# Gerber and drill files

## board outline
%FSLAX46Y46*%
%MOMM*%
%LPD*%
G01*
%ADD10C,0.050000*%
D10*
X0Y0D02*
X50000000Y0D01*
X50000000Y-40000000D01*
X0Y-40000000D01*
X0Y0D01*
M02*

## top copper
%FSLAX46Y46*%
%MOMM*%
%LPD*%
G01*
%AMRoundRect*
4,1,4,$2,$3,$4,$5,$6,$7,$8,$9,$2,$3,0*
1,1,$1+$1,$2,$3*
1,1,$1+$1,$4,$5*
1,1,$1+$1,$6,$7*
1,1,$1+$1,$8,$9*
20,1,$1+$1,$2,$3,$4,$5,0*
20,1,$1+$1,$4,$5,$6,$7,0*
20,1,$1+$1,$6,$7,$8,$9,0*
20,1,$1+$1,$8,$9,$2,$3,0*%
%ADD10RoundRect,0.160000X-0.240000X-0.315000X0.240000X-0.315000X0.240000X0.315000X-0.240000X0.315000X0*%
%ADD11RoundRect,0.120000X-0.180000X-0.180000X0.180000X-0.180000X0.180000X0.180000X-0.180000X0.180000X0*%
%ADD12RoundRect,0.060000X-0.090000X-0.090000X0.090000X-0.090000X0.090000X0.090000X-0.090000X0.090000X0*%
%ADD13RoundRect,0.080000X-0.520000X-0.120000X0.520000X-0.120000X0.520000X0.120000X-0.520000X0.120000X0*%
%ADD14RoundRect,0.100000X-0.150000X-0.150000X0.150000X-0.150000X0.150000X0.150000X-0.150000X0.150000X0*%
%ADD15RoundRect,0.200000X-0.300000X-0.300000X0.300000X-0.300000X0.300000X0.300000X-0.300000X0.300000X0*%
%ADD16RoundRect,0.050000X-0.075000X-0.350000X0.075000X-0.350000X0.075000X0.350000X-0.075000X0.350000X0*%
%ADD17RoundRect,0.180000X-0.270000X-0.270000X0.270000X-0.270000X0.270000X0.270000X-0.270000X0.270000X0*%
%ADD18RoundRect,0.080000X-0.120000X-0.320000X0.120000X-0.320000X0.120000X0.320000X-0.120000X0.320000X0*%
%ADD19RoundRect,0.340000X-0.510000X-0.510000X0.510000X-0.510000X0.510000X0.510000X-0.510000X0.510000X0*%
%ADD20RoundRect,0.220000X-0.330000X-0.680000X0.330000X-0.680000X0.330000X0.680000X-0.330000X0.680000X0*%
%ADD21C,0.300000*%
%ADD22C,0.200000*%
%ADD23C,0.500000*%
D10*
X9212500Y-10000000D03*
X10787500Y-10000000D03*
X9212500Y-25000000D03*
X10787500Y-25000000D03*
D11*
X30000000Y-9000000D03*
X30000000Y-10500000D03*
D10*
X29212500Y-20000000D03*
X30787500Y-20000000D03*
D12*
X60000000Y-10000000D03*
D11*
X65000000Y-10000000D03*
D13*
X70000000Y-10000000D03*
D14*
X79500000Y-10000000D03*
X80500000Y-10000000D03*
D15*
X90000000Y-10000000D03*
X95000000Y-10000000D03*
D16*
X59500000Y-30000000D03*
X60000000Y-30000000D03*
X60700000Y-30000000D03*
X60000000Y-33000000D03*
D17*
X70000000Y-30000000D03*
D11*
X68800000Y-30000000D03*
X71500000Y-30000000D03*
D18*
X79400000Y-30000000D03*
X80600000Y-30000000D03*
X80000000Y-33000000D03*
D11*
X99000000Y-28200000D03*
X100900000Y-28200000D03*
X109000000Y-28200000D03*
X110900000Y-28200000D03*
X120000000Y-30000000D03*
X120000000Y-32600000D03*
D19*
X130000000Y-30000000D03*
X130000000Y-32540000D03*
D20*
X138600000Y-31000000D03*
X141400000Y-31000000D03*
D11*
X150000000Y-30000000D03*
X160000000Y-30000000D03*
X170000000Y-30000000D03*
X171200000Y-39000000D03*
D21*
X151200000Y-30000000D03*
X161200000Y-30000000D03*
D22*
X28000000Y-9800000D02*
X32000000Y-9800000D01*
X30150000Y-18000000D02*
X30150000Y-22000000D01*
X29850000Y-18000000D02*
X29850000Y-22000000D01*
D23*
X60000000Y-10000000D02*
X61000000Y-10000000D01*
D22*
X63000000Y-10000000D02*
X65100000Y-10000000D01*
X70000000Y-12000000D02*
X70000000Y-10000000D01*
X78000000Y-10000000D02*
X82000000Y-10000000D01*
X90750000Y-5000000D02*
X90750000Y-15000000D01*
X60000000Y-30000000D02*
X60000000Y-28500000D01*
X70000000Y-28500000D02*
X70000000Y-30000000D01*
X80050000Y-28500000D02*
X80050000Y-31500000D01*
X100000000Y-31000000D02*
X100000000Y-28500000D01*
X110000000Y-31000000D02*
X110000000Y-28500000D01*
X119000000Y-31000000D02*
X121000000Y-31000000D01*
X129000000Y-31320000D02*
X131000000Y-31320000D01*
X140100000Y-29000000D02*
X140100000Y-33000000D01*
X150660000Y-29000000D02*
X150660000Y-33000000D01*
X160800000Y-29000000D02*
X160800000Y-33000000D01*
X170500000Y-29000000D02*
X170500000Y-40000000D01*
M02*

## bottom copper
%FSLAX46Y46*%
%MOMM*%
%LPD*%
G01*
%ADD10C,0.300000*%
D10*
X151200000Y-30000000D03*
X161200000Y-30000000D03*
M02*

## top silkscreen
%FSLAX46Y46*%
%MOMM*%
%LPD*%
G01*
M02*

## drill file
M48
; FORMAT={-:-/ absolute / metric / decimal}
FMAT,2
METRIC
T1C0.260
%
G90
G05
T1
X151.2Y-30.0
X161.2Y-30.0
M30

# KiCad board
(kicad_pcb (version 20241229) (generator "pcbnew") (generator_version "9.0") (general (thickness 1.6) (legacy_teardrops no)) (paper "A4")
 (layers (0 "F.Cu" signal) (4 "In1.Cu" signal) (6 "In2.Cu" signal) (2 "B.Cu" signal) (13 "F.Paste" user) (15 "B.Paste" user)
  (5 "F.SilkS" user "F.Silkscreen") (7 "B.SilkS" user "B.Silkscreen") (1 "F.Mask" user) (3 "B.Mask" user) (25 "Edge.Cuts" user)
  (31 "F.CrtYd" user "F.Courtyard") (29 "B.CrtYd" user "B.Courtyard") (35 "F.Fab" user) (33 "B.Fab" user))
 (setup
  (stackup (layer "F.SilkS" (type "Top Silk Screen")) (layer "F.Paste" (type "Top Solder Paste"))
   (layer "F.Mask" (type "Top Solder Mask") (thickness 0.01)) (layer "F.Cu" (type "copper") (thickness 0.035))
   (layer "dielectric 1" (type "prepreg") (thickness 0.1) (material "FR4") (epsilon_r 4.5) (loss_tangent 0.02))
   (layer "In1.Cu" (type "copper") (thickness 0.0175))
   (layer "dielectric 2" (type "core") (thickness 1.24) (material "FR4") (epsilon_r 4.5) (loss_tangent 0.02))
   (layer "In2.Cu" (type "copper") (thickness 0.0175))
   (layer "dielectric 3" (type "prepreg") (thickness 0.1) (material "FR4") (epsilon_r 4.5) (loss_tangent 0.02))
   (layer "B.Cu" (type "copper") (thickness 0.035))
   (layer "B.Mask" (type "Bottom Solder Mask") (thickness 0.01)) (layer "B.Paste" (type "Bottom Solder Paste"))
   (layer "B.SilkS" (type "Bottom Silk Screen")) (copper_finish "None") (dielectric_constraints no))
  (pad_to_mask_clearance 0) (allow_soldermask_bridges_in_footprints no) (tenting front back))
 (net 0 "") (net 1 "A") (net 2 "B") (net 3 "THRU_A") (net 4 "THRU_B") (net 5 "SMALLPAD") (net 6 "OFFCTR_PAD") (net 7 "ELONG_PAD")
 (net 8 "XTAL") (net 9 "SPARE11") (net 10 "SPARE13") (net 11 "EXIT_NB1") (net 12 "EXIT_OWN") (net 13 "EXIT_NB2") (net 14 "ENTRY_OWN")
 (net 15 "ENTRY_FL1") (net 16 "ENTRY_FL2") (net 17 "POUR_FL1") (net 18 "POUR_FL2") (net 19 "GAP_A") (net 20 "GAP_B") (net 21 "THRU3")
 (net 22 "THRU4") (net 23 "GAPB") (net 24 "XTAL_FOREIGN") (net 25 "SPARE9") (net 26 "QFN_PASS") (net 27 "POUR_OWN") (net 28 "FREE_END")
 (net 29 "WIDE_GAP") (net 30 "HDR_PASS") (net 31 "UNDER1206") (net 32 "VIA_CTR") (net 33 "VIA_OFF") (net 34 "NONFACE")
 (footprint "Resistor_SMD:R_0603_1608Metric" (layer "F.Cu") (at 10 10)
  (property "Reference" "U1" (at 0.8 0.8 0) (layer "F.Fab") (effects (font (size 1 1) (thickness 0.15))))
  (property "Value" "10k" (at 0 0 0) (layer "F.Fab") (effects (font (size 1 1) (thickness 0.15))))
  (pad "1" smd roundrect (at -0.7875 0) (size 0.8 0.95) (layers "F.Cu" "F.Paste" "F.Mask") (roundrect_rratio 0.2) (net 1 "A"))
  (pad "2" smd roundrect (at 0.7875 0) (size 0.8 0.95) (layers "F.Cu" "F.Paste" "F.Mask") (roundrect_rratio 0.2) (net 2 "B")))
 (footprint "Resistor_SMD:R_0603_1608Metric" (layer "F.Cu") (at 10 25)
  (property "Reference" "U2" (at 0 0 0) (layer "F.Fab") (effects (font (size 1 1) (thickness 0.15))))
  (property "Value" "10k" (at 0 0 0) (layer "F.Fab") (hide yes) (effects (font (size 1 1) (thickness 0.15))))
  (pad "1" smd roundrect (at -0.7875 0) (size 0.8 0.95) (layers "F.Cu" "F.Paste" "F.Mask") (roundrect_rratio 0.2) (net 1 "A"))
  (pad "2" smd roundrect (at 0.7875 0) (size 0.8 0.95) (layers "F.Cu" "F.Paste" "F.Mask") (roundrect_rratio 0.2) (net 2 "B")))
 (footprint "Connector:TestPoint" (layer "F.Cu") (at 30 9)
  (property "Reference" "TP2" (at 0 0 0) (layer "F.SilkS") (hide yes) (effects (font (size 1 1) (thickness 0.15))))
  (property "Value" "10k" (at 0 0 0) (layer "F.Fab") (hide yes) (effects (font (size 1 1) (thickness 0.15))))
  (pad "1" smd roundrect (at 0 0) (size 0.6 0.6) (layers "F.Cu" "F.Paste" "F.Mask") (roundrect_rratio 0.2) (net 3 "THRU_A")))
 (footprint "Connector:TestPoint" (layer "F.Cu") (at 30 10.5)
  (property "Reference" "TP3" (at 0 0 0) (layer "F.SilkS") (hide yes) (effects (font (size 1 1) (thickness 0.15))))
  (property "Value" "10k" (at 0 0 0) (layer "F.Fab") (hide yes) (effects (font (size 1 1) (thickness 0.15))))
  (pad "1" smd roundrect (at 0 0) (size 0.6 0.6) (layers "F.Cu" "F.Paste" "F.Mask") (roundrect_rratio 0.2) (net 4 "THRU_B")))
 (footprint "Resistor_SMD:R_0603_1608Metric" (layer "F.Cu") (at 30 20)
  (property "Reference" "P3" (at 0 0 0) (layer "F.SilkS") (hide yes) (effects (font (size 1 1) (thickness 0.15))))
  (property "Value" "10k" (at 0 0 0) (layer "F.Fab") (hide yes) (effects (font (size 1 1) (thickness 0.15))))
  (pad "1" smd roundrect (at -0.7875 0) (size 0.8 0.95) (layers "F.Cu" "F.Paste" "F.Mask") (roundrect_rratio 0.2) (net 1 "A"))
  (pad "2" smd roundrect (at 0.7875 0) (size 0.8 0.95) (layers "F.Cu" "F.Paste" "F.Mask") (roundrect_rratio 0.2) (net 2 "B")))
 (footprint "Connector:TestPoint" (layer "F.Cu") (at 60 10)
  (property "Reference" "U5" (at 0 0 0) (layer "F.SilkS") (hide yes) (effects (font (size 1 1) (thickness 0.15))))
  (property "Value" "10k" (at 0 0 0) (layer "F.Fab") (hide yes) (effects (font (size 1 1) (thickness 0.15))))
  (pad "1" smd roundrect (at 0 0) (size 0.3 0.3) (layers "F.Cu" "F.Paste" "F.Mask") (roundrect_rratio 0.2) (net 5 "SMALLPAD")))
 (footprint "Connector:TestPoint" (layer "F.Cu") (at 65 10)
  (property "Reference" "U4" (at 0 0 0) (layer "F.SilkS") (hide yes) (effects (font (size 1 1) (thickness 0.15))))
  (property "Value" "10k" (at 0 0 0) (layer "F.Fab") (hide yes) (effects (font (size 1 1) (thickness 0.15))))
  (pad "1" smd roundrect (at 0 0) (size 0.6 0.6) (layers "F.Cu" "F.Paste" "F.Mask") (roundrect_rratio 0.2) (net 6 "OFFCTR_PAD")))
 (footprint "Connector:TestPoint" (layer "F.Cu") (at 70 10)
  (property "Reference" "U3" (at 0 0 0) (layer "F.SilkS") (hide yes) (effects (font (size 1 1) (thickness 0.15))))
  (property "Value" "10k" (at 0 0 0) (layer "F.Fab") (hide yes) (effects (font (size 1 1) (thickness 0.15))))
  (pad "1" smd roundrect (at 0 0) (size 1.2 0.4) (layers "F.Cu" "F.Paste" "F.Mask") (roundrect_rratio 0.2) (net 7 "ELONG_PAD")))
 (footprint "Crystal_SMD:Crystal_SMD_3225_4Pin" (layer "F.Cu") (at 80 10)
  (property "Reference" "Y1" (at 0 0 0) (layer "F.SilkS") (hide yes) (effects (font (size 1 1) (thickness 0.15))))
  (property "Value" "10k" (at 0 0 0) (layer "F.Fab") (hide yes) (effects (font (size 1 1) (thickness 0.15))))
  (pad "1" smd roundrect (at -0.5 0) (size 0.5 0.5) (layers "F.Cu" "F.Paste" "F.Mask") (roundrect_rratio 0.2) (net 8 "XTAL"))
  (pad "2" smd roundrect (at 0.5 0) (size 0.5 0.5) (layers "F.Cu" "F.Paste" "F.Mask") (roundrect_rratio 0.2) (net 8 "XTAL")))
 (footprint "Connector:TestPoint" (layer "F.Cu") (at 90 10)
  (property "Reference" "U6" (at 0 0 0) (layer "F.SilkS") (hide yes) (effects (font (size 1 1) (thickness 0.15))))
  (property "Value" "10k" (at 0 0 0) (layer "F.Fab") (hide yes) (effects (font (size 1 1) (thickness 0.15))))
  (pad "1" smd roundrect (at 0 0) (size 1 1) (layers "F.Cu" "F.Paste" "F.Mask") (roundrect_rratio 0.2) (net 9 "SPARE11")))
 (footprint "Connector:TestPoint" (layer "F.Cu") (at 95 10)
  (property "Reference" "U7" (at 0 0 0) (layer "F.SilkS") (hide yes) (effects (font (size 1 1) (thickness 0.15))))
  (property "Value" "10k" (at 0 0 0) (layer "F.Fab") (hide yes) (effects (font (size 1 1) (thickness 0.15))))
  (pad "1" smd roundrect (at 0 0) (size 1 1) (layers "F.Cu" "F.Paste" "F.Mask") (roundrect_rratio 0.2) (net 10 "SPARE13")))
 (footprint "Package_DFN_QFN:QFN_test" (layer "F.Cu") (at 60 30)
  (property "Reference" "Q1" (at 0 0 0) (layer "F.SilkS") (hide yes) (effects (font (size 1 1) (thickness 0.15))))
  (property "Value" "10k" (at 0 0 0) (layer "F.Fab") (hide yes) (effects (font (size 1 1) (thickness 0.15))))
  (pad "1" smd roundrect (at -0.5 0) (size 0.25 0.8) (layers "F.Cu" "F.Paste" "F.Mask") (roundrect_rratio 0.2) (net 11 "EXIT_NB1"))
  (pad "2" smd roundrect (at 0 0) (size 0.25 0.8) (layers "F.Cu" "F.Paste" "F.Mask") (roundrect_rratio 0.2) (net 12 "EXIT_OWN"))
  (pad "3" smd roundrect (at 0.7 0) (size 0.25 0.8) (layers "F.Cu" "F.Paste" "F.Mask") (roundrect_rratio 0.2) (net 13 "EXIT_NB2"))
  (pad "4" smd roundrect (at 0 3) (size 0.25 0.8) (layers "F.Cu" "F.Paste" "F.Mask") (roundrect_rratio 0.2) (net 13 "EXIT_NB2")))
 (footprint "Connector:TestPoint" (layer "F.Cu") (at 70 30)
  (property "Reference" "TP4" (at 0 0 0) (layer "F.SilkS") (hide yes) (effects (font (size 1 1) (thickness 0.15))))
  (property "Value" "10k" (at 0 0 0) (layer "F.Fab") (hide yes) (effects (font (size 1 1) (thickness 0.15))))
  (pad "1" smd roundrect (at 0 0) (size 0.9 0.9) (layers "F.Cu" "F.Paste" "F.Mask") (roundrect_rratio 0.2) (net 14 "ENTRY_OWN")))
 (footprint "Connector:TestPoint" (layer "F.Cu") (at 68.8 30)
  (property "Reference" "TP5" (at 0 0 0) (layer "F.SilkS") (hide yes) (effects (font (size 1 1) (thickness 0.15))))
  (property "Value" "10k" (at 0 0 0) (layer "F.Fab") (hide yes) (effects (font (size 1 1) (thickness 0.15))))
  (pad "1" smd roundrect (at 0 0) (size 0.6 0.6) (layers "F.Cu" "F.Paste" "F.Mask") (roundrect_rratio 0.2) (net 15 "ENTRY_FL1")))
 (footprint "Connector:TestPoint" (layer "F.Cu") (at 71.5 30)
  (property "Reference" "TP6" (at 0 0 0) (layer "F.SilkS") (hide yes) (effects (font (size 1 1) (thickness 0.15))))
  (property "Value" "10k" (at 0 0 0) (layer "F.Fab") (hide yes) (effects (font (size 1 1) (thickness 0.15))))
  (pad "1" smd roundrect (at 0 0) (size 0.6 0.6) (layers "F.Cu" "F.Paste" "F.Mask") (roundrect_rratio 0.2) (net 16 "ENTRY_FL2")))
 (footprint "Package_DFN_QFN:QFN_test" (layer "F.Cu") (at 80 30)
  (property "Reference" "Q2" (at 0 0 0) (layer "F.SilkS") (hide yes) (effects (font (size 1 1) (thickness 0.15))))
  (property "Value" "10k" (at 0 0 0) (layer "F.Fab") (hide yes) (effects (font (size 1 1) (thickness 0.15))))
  (pad "1" smd roundrect (at -0.6 0) (size 0.4 0.8) (layers "F.Cu" "F.Paste" "F.Mask") (roundrect_rratio 0.2) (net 11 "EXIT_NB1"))
  (pad "2" smd roundrect (at 0.6 0) (size 0.4 0.8) (layers "F.Cu" "F.Paste" "F.Mask") (roundrect_rratio 0.2) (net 13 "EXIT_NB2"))
  (pad "3" smd roundrect (at 0 3) (size 0.4 0.8) (layers "F.Cu" "F.Paste" "F.Mask") (roundrect_rratio 0.2) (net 13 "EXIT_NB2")))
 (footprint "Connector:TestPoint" (layer "F.Cu") (at 99 28.2)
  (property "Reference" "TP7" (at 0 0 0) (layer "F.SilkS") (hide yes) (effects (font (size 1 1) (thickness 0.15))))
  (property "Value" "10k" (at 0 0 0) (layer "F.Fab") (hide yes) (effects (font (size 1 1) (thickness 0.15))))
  (pad "1" smd roundrect (at 0 0) (size 0.6 0.6) (layers "F.Cu" "F.Paste" "F.Mask") (roundrect_rratio 0.2) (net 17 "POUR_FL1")))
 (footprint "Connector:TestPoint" (layer "F.Cu") (at 100.9 28.2)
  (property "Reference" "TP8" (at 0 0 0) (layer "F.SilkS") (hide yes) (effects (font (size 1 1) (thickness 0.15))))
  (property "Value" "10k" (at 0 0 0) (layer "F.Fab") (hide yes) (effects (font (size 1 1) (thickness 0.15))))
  (pad "1" smd roundrect (at 0 0) (size 0.6 0.6) (layers "F.Cu" "F.Paste" "F.Mask") (roundrect_rratio 0.2) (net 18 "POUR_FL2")))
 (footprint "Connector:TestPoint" (layer "F.Cu") (at 109 28.2)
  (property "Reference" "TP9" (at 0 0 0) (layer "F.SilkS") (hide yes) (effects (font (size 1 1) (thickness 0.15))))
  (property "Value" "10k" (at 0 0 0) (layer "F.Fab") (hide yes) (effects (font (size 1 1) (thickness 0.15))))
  (pad "1" smd roundrect (at 0 0) (size 0.6 0.6) (layers "F.Cu" "F.Paste" "F.Mask") (roundrect_rratio 0.2) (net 17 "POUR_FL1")))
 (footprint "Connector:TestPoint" (layer "F.Cu") (at 110.9 28.2)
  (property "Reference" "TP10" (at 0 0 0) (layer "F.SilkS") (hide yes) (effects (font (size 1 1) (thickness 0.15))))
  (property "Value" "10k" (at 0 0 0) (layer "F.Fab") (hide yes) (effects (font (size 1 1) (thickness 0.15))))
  (pad "1" smd roundrect (at 0 0) (size 0.6 0.6) (layers "F.Cu" "F.Paste" "F.Mask") (roundrect_rratio 0.2) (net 18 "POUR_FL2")))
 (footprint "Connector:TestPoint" (layer "F.Cu") (at 120 30)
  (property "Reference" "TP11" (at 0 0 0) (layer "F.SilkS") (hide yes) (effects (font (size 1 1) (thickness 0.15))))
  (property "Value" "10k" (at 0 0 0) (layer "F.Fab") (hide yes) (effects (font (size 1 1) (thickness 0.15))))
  (pad "1" smd roundrect (at 0 0) (size 0.6 0.6) (layers "F.Cu" "F.Paste" "F.Mask") (roundrect_rratio 0.2) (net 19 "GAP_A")))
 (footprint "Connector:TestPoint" (layer "F.Cu") (at 120 32.6)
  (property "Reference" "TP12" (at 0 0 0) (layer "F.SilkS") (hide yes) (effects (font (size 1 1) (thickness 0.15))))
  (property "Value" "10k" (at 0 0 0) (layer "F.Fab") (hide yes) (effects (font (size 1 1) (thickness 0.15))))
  (pad "1" smd roundrect (at 0 0) (size 0.6 0.6) (layers "F.Cu" "F.Paste" "F.Mask") (roundrect_rratio 0.2) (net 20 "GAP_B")))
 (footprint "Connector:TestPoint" (layer "F.Cu") (at 130 30)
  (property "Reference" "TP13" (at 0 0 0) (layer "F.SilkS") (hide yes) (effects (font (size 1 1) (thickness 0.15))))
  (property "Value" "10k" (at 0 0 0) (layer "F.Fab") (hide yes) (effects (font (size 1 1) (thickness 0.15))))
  (pad "1" smd roundrect (at 0 0) (size 1.7 1.7) (layers "F.Cu" "F.Paste" "F.Mask") (roundrect_rratio 0.2) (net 19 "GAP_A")))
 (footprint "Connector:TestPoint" (layer "F.Cu") (at 130 32.54)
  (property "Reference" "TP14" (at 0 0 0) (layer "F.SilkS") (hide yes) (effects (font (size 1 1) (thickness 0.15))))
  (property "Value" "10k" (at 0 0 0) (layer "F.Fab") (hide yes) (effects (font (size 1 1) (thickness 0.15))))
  (pad "1" smd roundrect (at 0 0) (size 1.7 1.7) (layers "F.Cu" "F.Paste" "F.Mask") (roundrect_rratio 0.2) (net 20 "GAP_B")))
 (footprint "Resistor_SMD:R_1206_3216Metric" (layer "F.Cu") (at 140 31)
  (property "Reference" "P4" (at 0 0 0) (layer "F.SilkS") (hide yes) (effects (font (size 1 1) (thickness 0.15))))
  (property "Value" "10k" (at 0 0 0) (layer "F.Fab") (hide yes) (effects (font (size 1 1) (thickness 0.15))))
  (pad "1" smd roundrect (at -1.4 0) (size 1.1 1.8) (layers "F.Cu" "F.Paste" "F.Mask") (roundrect_rratio 0.2) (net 19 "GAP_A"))
  (pad "2" smd roundrect (at 1.4 0) (size 1.1 1.8) (layers "F.Cu" "F.Paste" "F.Mask") (roundrect_rratio 0.2) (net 20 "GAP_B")))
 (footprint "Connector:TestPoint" (layer "F.Cu") (at 150 30)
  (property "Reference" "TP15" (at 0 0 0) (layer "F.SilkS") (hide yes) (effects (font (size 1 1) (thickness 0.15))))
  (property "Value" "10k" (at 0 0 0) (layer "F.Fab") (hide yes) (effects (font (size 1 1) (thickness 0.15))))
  (pad "1" smd roundrect (at 0 0) (size 0.6 0.6) (layers "F.Cu" "F.Paste" "F.Mask") (roundrect_rratio 0.2) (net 19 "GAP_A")))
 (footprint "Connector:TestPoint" (layer "F.Cu") (at 160 30)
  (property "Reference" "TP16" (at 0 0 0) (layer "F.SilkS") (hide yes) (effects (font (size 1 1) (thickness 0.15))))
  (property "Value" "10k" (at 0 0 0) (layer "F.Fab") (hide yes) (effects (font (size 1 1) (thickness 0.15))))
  (pad "1" smd roundrect (at 0 0) (size 0.6 0.6) (layers "F.Cu" "F.Paste" "F.Mask") (roundrect_rratio 0.2) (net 19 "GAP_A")))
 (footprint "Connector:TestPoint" (layer "F.Cu") (at 170 30)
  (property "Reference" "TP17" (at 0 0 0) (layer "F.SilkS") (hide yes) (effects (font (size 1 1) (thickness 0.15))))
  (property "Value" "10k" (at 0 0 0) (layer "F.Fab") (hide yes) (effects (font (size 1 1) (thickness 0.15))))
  (pad "1" smd roundrect (at 0 0) (size 0.6 0.6) (layers "F.Cu" "F.Paste" "F.Mask") (roundrect_rratio 0.2) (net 19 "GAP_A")))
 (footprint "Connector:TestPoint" (layer "F.Cu") (at 171.2 39)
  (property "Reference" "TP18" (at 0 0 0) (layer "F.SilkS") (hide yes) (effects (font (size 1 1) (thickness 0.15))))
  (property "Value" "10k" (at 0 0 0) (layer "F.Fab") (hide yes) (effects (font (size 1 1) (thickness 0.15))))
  (pad "1" smd roundrect (at 0 0) (size 0.6 0.6) (layers "F.Cu" "F.Paste" "F.Mask") (roundrect_rratio 0.2) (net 20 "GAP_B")))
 (segment (start 28 9.8) (end 32 9.8) (width 0.2) (layer "F.Cu") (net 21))
 (segment (start 30.15 18) (end 30.15 22) (width 0.2) (layer "F.Cu") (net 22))
 (segment (start 29.85 18) (end 29.85 22) (width 0.2) (layer "F.Cu") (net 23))
 (segment (start 60 10) (end 61 10) (width 0.5) (layer "F.Cu") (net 5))
 (segment (start 63 10) (end 65.1 10) (width 0.2) (layer "F.Cu") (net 6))
 (segment (start 70 12) (end 70 10) (width 0.2) (layer "F.Cu") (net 7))
 (segment (start 78 10) (end 82 10) (width 0.2) (layer "F.Cu") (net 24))
 (segment (start 90.75 5) (end 90.75 15) (width 0.2) (layer "F.Cu") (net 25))
 (segment (start 60 30) (end 60 28.5) (width 0.2) (layer "F.Cu") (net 12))
 (segment (start 70 28.5) (end 70 30) (width 0.2) (layer "F.Cu") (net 14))
 (segment (start 80.05 28.5) (end 80.05 31.5) (width 0.2) (layer "F.Cu") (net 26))
 (segment (start 100 31) (end 100 28.5) (width 0.2) (layer "F.Cu") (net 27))
 (segment (start 110 31) (end 110 28.5) (width 0.2) (layer "F.Cu") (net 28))
 (segment (start 119 31) (end 121 31) (width 0.2) (layer "F.Cu") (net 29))
 (segment (start 129 31.32) (end 131 31.32) (width 0.2) (layer "F.Cu") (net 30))
 (segment (start 140.1 29) (end 140.1 33) (width 0.2) (layer "F.Cu") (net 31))
 (via (at 151.2 30) (size 0.3) (drill 0.26) (layers "F.Cu" "B.Cu") (remove_unused_layers yes) (keep_end_layers yes) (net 20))
 (segment (start 150.66 29) (end 150.66 33) (width 0.2) (layer "F.Cu") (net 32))
 (via (at 161.2 30) (size 0.3) (drill 0.26) (layers "F.Cu" "B.Cu") (remove_unused_layers yes) (keep_end_layers yes) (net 20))
 (segment (start 160.8 29) (end 160.8 33) (width 0.2) (layer "F.Cu") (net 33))
 (segment (start 170.5 29) (end 170.5 40) (width 0.2) (layer "F.Cu") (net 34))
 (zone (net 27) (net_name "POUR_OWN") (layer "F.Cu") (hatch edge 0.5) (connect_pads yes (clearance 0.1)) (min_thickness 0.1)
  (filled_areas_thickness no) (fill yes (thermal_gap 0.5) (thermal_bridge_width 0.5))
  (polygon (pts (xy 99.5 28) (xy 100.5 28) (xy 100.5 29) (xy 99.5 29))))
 (gr_rect (start 0 0) (end 50 40) (stroke (width 0.05) (type default)) (fill no) (layer "Edge.Cuts")))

